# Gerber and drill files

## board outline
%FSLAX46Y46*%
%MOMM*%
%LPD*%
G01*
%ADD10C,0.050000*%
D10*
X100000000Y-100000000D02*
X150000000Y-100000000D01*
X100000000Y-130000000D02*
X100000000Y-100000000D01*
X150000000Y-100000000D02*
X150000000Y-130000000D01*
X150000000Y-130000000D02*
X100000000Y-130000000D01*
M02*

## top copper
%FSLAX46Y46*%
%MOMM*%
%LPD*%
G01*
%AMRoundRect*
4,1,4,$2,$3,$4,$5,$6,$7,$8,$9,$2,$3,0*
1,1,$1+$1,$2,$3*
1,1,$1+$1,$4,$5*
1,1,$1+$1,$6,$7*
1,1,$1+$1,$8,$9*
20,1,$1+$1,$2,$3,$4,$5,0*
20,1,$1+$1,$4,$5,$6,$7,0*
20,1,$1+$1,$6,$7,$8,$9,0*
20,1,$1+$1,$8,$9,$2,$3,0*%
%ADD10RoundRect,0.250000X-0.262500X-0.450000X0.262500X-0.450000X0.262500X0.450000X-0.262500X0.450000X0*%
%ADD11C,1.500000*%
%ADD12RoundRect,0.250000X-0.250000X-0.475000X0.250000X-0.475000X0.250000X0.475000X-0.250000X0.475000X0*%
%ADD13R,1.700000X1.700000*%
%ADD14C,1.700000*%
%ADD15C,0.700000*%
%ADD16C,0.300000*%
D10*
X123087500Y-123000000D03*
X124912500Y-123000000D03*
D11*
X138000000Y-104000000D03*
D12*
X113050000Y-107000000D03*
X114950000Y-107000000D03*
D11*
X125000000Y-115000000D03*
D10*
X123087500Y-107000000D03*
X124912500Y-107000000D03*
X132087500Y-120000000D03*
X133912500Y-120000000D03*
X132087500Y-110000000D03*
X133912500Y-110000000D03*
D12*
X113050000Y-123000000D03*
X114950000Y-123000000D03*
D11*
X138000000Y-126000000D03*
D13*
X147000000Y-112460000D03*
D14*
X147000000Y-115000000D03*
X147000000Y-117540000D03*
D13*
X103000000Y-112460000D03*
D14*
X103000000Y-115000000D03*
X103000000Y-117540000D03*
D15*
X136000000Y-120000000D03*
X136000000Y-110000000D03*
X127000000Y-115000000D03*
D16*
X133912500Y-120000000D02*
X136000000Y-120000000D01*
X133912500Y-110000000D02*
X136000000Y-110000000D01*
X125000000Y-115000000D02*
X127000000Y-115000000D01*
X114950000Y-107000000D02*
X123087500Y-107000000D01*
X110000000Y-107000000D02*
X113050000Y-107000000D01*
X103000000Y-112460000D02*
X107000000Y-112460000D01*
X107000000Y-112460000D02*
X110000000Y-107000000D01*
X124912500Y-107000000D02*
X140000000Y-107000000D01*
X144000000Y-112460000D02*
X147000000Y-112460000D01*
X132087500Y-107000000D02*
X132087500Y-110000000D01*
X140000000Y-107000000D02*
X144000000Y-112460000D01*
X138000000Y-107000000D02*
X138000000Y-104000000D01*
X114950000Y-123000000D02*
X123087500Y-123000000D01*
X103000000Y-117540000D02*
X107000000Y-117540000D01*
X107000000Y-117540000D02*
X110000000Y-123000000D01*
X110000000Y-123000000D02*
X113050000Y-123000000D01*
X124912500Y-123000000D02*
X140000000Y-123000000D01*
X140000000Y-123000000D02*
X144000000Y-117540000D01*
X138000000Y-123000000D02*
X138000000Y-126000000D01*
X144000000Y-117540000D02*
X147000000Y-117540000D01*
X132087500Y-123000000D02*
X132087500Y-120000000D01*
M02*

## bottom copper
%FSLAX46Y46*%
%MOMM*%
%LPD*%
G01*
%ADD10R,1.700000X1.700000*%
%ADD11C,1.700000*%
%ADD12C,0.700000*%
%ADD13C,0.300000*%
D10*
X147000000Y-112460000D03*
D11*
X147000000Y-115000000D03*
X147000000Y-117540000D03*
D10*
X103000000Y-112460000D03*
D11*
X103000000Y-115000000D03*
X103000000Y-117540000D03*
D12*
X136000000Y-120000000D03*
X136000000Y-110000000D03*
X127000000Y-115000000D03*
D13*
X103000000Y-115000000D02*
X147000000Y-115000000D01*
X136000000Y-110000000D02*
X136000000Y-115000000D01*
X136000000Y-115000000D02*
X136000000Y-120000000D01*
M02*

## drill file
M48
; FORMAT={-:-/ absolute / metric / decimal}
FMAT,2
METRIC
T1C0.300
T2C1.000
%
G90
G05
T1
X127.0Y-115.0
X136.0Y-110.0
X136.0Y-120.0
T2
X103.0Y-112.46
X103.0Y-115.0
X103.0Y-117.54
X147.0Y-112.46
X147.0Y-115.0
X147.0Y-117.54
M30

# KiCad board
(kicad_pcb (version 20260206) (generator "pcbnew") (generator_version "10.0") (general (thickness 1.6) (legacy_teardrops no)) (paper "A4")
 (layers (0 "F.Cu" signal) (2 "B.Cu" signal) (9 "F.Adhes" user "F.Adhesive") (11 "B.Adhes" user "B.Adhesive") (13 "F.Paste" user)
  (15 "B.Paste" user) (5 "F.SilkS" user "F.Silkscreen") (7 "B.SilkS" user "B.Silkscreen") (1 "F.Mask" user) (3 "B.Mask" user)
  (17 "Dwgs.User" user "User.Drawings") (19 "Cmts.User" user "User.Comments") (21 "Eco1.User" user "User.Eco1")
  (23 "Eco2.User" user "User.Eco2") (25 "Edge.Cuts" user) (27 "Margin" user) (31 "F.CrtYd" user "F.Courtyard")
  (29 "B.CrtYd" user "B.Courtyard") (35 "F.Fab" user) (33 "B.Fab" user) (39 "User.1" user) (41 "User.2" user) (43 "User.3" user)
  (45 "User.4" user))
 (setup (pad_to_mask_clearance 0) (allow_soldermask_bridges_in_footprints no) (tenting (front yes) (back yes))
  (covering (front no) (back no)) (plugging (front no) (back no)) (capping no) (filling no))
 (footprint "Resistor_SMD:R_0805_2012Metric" (layer "F.Cu") (at 124 123)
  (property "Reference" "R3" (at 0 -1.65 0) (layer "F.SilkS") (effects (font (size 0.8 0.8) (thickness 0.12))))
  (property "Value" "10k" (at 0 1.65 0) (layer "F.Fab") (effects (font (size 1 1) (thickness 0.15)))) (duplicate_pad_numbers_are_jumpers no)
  (pad "1" smd roundrect (at -0.9125 0) (size 1.025 1.4) (layers "F.Cu" "F.Mask" "F.Paste") (roundrect_rratio 0.243902) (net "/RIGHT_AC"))
  (pad "2" smd roundrect (at 0.9125 0) (size 1.025 1.4) (layers "F.Cu" "F.Mask" "F.Paste") (roundrect_rratio 0.243902) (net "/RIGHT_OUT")))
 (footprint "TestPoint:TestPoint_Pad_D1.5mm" (layer "F.Cu") (at 138 104)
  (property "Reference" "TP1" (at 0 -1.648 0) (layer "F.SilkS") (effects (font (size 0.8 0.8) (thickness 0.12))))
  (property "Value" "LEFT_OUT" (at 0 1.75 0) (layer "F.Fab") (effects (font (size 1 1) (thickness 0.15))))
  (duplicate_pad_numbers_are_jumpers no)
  (pad "1" smd circle (at 0 0) (size 1.5 1.5) (layers "F.Cu" "F.Mask") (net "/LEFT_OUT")))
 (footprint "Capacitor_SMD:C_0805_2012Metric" (layer "F.Cu") (at 114 107)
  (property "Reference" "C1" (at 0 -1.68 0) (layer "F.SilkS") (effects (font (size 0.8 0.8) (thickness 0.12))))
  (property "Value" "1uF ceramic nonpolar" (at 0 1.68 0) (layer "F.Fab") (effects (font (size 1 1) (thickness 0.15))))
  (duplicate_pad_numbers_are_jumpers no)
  (pad "1" smd roundrect (at -0.95 0) (size 1 1.45) (layers "F.Cu" "F.Mask" "F.Paste") (roundrect_rratio 0.25) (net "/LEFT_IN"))
  (pad "2" smd roundrect (at 0.95 0) (size 1 1.45) (layers "F.Cu" "F.Mask" "F.Paste") (roundrect_rratio 0.25) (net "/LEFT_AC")))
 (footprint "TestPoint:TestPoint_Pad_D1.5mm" (layer "F.Cu") (at 125 115)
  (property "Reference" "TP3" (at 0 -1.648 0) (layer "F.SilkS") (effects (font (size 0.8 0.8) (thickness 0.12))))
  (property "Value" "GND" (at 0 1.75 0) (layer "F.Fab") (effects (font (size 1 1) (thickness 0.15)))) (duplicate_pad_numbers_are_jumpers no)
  (pad "1" smd circle (at 0 0) (size 1.5 1.5) (layers "F.Cu" "F.Mask") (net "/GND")))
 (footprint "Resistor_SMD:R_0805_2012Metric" (layer "F.Cu") (at 124 107)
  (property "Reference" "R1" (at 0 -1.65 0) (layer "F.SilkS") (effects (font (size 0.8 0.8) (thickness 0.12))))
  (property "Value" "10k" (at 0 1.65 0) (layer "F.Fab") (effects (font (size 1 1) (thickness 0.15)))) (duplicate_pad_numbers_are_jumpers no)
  (pad "1" smd roundrect (at -0.9125 0) (size 1.025 1.4) (layers "F.Cu" "F.Mask" "F.Paste") (roundrect_rratio 0.243902) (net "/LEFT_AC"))
  (pad "2" smd roundrect (at 0.9125 0) (size 1.025 1.4) (layers "F.Cu" "F.Mask" "F.Paste") (roundrect_rratio 0.243902) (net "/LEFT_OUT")))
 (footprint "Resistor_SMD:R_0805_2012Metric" (layer "F.Cu") (at 133 120)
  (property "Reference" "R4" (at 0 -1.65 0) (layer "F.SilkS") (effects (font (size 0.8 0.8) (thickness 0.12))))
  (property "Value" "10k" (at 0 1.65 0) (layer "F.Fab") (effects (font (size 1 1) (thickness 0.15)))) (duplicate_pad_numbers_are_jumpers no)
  (pad "1" smd roundrect (at -0.9125 0) (size 1.025 1.4) (layers "F.Cu" "F.Mask" "F.Paste") (roundrect_rratio 0.243902) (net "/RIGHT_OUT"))
  (pad "2" smd roundrect (at 0.9125 0) (size 1.025 1.4) (layers "F.Cu" "F.Mask" "F.Paste") (roundrect_rratio 0.243902) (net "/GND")))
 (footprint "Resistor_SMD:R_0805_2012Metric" (layer "F.Cu") (at 133 110)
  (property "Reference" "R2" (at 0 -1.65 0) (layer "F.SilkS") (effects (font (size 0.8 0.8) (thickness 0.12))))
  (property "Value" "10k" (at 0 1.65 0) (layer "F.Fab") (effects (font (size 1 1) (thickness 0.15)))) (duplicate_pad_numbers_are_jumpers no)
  (pad "1" smd roundrect (at -0.9125 0) (size 1.025 1.4) (layers "F.Cu" "F.Mask" "F.Paste") (roundrect_rratio 0.243902) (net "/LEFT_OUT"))
  (pad "2" smd roundrect (at 0.9125 0) (size 1.025 1.4) (layers "F.Cu" "F.Mask" "F.Paste") (roundrect_rratio 0.243902) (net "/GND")))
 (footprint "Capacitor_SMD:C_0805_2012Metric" (layer "F.Cu") (at 114 123)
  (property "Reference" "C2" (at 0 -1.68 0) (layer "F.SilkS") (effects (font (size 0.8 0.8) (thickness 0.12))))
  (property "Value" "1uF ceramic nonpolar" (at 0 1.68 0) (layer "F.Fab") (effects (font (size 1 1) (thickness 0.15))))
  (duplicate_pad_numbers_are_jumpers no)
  (pad "1" smd roundrect (at -0.95 0) (size 1 1.45) (layers "F.Cu" "F.Mask" "F.Paste") (roundrect_rratio 0.25) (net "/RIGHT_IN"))
  (pad "2" smd roundrect (at 0.95 0) (size 1 1.45) (layers "F.Cu" "F.Mask" "F.Paste") (roundrect_rratio 0.25) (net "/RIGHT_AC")))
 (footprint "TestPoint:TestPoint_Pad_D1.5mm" (layer "F.Cu") (at 138 126)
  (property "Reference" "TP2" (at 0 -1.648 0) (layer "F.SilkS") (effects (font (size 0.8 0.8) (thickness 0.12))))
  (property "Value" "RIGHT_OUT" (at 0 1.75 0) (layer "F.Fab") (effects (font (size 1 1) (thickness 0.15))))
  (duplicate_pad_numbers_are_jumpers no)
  (pad "1" smd circle (at 0 0) (size 1.5 1.5) (layers "F.Cu" "F.Mask") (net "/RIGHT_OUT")))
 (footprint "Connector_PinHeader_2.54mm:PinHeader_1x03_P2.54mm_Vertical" (layer "F.Cu") (at 147 112.46)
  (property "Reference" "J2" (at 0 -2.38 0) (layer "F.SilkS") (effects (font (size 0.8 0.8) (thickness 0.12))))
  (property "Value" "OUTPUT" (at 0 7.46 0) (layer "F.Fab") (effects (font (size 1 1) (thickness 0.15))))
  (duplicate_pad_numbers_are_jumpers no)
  (pad "1" thru_hole rect (at 0 0) (size 1.7 1.7) (drill 1) (layers "*.Cu" "*.Mask") (remove_unused_layers no) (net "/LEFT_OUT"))
  (pad "2" thru_hole circle (at 0 2.54) (size 1.7 1.7) (drill 1) (layers "*.Cu" "*.Mask") (remove_unused_layers no) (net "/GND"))
  (pad "3" thru_hole circle (at 0 5.08) (size 1.7 1.7) (drill 1) (layers "*.Cu" "*.Mask") (remove_unused_layers no) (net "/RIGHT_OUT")))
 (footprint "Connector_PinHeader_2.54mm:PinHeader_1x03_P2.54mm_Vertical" (layer "F.Cu") (at 103 112.46)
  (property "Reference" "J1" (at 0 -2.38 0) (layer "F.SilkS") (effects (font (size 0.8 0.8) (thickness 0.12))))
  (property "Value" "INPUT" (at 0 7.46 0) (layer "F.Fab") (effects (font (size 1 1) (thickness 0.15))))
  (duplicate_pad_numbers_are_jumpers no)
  (pad "1" thru_hole rect (at 0 0) (size 1.7 1.7) (drill 1) (layers "*.Cu" "*.Mask") (remove_unused_layers no) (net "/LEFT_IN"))
  (pad "2" thru_hole circle (at 0 2.54) (size 1.7 1.7) (drill 1) (layers "*.Cu" "*.Mask") (remove_unused_layers no) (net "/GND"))
  (pad "3" thru_hole circle (at 0 5.08) (size 1.7 1.7) (drill 1) (layers "*.Cu" "*.Mask") (remove_unused_layers no) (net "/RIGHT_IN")))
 (gr_line (start 100 100) (end 150 100) (stroke (width 0.05) (type default)) (layer "Edge.Cuts"))
 (gr_line (start 100 130) (end 100 100) (stroke (width 0.05) (type default)) (layer "Edge.Cuts"))
 (gr_line (start 150 100) (end 150 130) (stroke (width 0.05) (type default)) (layer "Edge.Cuts"))
 (gr_line (start 150 130) (end 100 130) (stroke (width 0.05) (type default)) (layer "Edge.Cuts"))
 (segment (start 133.9125 120) (end 136 120) (width 0.3) (layer "F.Cu") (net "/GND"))
 (segment (start 133.9125 110) (end 136 110) (width 0.3) (layer "F.Cu") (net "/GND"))
 (segment (start 125 115) (end 127 115) (width 0.3) (layer "F.Cu") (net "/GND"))
 (via (at 136 120) (size 0.7) (drill 0.3) (layers "F.Cu" "B.Cu") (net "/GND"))
 (via (at 136 110) (size 0.7) (drill 0.3) (layers "F.Cu" "B.Cu") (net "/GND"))
 (via (at 127 115) (size 0.7) (drill 0.3) (layers "F.Cu" "B.Cu") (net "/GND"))
 (segment (start 103 115) (end 147 115) (width 0.3) (layer "B.Cu") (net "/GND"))
 (segment (start 136 110) (end 136 115) (width 0.3) (layer "B.Cu") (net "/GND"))
 (segment (start 136 115) (end 136 120) (width 0.3) (layer "B.Cu") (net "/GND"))
 (segment (start 114.95 107) (end 123.0875 107) (width 0.3) (layer "F.Cu") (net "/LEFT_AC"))
 (segment (start 110 107) (end 113.05 107) (width 0.3) (layer "F.Cu") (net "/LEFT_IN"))
 (segment (start 103 112.46) (end 107 112.46) (width 0.3) (layer "F.Cu") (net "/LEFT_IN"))
 (segment (start 107 112.46) (end 110 107) (width 0.3) (layer "F.Cu") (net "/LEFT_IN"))
 (segment (start 124.9125 107) (end 140 107) (width 0.3) (layer "F.Cu") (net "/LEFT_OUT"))
 (segment (start 144 112.46) (end 147 112.46) (width 0.3) (layer "F.Cu") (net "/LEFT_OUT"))
 (segment (start 132.0875 107) (end 132.0875 110) (width 0.3) (layer "F.Cu") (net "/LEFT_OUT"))
 (segment (start 140 107) (end 144 112.46) (width 0.3) (layer "F.Cu") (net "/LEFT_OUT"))
 (segment (start 138 107) (end 138 104) (width 0.3) (layer "F.Cu") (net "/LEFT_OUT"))
 (segment (start 114.95 123) (end 123.0875 123) (width 0.3) (layer "F.Cu") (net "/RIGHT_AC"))
 (segment (start 103 117.54) (end 107 117.54) (width 0.3) (layer "F.Cu") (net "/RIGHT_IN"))
 (segment (start 107 117.54) (end 110 123) (width 0.3) (layer "F.Cu") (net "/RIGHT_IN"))
 (segment (start 110 123) (end 113.05 123) (width 0.3) (layer "F.Cu") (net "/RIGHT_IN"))
 (segment (start 124.9125 123) (end 140 123) (width 0.3) (layer "F.Cu") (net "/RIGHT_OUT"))
 (segment (start 140 123) (end 144 117.54) (width 0.3) (layer "F.Cu") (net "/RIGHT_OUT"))
 (segment (start 138 123) (end 138 126) (width 0.3) (layer "F.Cu") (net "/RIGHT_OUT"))
 (segment (start 144 117.54) (end 147 117.54) (width 0.3) (layer "F.Cu") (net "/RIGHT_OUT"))
 (segment (start 132.0875 123) (end 132.0875 120) (width 0.3) (layer "F.Cu") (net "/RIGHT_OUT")))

